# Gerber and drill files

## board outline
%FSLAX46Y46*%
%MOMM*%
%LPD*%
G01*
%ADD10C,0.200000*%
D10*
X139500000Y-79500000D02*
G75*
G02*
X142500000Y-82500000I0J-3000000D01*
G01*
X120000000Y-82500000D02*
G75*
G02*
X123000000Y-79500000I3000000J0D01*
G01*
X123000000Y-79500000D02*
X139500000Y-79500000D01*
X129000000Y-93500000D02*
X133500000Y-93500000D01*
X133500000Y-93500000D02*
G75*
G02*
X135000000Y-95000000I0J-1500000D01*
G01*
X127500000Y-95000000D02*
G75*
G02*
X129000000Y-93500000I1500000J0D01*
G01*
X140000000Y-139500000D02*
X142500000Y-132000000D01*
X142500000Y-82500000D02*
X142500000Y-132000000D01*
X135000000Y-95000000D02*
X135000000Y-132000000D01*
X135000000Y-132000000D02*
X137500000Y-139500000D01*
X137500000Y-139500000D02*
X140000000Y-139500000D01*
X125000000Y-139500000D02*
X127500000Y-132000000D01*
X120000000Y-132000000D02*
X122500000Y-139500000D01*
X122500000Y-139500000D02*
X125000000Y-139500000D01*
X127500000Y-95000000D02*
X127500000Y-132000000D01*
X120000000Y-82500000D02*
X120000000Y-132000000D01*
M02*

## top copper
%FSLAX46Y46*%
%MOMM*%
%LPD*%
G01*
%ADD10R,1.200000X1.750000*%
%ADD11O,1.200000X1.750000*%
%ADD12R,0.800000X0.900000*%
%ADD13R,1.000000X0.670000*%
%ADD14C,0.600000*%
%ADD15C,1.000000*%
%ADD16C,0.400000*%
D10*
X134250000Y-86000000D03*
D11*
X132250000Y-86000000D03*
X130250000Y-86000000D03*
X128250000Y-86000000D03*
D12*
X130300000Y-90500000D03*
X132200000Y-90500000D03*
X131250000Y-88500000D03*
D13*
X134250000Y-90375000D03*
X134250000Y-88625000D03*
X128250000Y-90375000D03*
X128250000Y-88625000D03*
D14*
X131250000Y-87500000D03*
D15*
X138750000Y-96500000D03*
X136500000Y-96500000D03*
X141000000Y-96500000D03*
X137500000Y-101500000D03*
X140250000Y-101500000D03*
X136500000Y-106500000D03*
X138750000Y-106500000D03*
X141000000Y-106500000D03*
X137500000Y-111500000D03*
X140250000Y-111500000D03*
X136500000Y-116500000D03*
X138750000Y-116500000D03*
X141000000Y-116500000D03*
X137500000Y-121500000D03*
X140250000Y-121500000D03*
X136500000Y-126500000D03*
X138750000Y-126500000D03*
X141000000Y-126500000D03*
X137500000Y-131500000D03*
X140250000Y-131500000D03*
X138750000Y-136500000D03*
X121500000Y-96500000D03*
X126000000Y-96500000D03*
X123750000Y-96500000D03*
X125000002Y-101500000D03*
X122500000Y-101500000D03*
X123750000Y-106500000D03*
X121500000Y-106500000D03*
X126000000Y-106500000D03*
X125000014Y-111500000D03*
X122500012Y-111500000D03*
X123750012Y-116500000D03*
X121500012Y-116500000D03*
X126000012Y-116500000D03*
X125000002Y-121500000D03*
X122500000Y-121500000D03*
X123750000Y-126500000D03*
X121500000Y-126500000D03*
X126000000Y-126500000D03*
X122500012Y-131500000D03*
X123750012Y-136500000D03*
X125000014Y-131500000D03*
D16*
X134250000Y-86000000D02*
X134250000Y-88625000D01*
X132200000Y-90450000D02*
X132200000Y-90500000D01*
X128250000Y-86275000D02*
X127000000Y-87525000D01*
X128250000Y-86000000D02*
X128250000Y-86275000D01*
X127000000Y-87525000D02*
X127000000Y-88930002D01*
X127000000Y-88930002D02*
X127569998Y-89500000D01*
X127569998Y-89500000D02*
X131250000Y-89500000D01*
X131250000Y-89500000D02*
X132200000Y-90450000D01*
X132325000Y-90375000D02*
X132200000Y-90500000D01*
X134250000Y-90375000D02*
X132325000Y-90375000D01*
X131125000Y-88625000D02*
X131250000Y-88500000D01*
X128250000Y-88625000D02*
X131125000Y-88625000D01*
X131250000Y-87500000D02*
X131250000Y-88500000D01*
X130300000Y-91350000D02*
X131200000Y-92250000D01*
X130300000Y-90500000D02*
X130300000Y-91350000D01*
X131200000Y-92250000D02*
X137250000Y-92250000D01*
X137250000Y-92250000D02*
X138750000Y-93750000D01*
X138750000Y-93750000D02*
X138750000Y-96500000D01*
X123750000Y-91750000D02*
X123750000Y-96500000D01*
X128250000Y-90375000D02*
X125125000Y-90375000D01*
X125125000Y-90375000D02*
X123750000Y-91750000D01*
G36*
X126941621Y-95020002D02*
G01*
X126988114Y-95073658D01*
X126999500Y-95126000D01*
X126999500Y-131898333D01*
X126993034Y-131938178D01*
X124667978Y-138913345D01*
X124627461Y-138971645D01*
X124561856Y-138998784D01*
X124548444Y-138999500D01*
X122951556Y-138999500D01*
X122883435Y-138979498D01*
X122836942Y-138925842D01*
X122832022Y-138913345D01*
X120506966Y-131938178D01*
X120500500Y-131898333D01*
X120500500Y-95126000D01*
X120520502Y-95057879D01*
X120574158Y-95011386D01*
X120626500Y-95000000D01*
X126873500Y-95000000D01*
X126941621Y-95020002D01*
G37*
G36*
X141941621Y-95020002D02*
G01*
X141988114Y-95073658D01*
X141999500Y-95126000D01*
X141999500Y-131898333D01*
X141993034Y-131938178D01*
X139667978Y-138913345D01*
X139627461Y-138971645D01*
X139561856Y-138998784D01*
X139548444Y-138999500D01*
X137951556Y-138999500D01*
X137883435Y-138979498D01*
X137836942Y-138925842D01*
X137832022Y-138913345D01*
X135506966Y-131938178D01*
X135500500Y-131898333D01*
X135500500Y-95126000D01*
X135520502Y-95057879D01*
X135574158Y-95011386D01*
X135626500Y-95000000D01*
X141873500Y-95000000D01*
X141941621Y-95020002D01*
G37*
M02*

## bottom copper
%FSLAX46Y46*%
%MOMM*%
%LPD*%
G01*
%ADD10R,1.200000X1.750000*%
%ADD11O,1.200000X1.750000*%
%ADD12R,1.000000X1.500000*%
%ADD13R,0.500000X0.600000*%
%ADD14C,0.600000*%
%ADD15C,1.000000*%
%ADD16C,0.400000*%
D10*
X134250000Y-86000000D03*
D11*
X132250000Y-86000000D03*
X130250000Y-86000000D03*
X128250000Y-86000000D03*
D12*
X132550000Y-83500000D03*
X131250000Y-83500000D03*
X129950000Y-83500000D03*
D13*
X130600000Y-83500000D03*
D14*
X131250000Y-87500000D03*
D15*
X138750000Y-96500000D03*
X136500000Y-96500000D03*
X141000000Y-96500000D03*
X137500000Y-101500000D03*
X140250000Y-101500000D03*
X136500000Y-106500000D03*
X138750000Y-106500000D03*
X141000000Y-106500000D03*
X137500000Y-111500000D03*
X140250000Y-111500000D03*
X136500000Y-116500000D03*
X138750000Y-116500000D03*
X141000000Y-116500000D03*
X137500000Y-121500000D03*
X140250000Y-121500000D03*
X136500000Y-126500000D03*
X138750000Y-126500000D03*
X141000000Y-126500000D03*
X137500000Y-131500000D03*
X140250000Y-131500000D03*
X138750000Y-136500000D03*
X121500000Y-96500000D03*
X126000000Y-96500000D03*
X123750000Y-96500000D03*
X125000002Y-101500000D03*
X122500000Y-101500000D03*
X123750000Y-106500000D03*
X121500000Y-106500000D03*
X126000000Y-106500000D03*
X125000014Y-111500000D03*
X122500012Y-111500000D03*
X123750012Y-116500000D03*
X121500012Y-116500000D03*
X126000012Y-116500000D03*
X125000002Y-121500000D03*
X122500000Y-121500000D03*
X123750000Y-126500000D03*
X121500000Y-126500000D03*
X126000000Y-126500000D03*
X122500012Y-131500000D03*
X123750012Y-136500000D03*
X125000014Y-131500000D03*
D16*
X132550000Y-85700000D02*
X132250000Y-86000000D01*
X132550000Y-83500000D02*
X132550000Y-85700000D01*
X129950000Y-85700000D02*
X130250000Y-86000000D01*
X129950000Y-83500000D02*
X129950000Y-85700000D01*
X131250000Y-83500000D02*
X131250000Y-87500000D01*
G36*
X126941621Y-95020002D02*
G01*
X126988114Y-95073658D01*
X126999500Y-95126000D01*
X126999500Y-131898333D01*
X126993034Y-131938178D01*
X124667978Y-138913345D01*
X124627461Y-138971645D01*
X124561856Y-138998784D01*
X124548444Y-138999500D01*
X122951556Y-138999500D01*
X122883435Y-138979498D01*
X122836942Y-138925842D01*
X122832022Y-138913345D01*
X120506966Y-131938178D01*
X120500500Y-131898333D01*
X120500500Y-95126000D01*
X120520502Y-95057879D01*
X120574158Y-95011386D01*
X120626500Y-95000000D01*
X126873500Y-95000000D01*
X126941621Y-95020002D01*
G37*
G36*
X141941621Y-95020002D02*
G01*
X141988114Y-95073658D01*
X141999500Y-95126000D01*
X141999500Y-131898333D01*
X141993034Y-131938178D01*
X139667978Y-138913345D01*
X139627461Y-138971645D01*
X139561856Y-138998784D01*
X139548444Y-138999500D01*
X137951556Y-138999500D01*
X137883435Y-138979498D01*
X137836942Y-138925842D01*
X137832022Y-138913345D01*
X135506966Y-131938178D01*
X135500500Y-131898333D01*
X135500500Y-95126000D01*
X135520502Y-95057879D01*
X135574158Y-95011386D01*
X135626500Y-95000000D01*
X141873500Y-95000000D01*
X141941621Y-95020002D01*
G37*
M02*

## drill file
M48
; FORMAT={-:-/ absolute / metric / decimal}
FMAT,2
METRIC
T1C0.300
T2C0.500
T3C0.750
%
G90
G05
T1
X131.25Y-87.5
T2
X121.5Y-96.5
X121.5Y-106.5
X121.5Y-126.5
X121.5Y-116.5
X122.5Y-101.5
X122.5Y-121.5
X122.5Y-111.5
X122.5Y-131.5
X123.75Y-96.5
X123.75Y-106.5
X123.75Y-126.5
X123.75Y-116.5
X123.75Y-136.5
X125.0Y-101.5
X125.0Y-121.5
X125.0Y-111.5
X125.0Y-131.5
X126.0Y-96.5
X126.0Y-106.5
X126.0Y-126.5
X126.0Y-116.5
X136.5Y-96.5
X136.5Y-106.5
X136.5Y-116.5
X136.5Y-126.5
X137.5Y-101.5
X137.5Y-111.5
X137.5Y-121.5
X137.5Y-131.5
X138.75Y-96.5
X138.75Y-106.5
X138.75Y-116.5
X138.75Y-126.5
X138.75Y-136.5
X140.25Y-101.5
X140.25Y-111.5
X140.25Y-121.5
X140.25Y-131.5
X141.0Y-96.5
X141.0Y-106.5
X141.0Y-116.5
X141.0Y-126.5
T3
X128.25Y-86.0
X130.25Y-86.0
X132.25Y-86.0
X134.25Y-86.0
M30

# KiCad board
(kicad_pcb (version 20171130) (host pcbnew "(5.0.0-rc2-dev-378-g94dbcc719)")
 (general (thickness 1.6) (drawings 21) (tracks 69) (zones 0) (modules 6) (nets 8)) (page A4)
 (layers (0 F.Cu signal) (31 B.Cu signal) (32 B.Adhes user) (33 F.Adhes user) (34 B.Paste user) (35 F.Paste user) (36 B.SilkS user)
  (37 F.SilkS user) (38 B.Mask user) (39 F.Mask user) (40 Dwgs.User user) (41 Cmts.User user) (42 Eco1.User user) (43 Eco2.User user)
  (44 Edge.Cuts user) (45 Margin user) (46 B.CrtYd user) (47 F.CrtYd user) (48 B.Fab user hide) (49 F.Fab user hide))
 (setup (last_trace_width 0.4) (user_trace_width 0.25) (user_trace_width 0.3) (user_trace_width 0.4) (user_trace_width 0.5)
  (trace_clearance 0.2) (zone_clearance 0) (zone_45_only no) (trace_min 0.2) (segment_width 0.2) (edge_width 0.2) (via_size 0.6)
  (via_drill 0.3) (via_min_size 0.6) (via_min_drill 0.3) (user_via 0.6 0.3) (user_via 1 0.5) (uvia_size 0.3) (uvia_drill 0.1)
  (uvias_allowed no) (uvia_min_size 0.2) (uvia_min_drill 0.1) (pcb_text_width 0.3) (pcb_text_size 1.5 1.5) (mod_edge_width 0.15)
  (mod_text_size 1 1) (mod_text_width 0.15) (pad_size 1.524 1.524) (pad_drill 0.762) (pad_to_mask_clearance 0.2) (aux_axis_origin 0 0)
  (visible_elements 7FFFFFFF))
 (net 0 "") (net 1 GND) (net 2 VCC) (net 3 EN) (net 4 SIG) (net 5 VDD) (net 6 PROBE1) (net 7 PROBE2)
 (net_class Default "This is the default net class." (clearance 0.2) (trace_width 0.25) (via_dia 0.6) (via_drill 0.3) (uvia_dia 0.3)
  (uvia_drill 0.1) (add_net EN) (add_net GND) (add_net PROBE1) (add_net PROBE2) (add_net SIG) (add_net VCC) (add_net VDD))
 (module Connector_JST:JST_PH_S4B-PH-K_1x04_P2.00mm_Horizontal (layer F.Cu) (at 134.25 86 180)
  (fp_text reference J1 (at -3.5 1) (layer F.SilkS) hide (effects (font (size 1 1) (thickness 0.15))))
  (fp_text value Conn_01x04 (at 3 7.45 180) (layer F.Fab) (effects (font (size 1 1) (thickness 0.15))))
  (pad 1 thru_hole rect (at 0 0 180) (size 1.2 1.75) (drill 0.75) (layers *.Cu *.Mask) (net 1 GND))
  (pad 2 thru_hole oval (at 2 0 180) (size 1.2 1.75) (drill 0.75) (layers *.Cu *.Mask) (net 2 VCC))
  (pad 3 thru_hole oval (at 4 0 180) (size 1.2 1.75) (drill 0.75) (layers *.Cu *.Mask) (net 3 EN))
  (pad 4 thru_hole oval (at 6 0 180) (size 1.2 1.75) (drill 0.75) (layers *.Cu *.Mask) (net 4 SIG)))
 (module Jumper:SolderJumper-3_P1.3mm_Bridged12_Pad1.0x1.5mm (layer B.Cu) (at 131.25 83.5)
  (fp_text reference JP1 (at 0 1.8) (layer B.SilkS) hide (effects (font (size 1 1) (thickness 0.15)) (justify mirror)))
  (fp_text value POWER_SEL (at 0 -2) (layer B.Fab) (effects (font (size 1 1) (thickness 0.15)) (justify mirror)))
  (pad 3 smd rect (at 1.3 0) (size 1 1.5) (layers B.Cu B.Mask) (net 2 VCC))
  (pad 2 smd rect (at 0 0) (size 1 1.5) (layers B.Cu B.Mask) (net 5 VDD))
  (pad 1 smd rect (at -1.3 0) (size 1 1.5) (layers B.Cu B.Mask) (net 3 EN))
  (pad 1 smd rect (at -0.65 0) (size 0.5 0.6) (layers B.Cu B.Mask) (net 3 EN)))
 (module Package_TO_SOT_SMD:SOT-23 (layer F.Cu) (at 131.25 89.5 90)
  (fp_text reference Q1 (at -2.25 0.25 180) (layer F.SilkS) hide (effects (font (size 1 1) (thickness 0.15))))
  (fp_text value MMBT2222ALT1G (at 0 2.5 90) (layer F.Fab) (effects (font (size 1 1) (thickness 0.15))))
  (pad 1 smd rect (at -1 -0.95 90) (size 0.9 0.8) (layers F.Cu F.Paste F.Mask) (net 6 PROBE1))
  (pad 2 smd rect (at -1 0.95 90) (size 0.9 0.8) (layers F.Cu F.Paste F.Mask) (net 4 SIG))
  (pad 3 smd rect (at 1 0 90) (size 0.9 0.8) (layers F.Cu F.Paste F.Mask) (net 5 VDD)))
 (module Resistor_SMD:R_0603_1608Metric (layer F.Cu) (at 134.25 89.5 90)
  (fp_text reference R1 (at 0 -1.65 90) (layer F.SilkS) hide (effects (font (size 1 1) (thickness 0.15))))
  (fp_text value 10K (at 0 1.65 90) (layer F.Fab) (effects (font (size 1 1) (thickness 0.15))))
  (pad 1 smd rect (at -0.875 0 90) (size 0.67 1) (layers F.Cu F.Paste F.Mask) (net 4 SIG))
  (pad 2 smd rect (at 0.875 0 90) (size 0.67 1) (layers F.Cu F.Paste F.Mask) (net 1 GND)))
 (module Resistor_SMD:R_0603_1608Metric (layer F.Cu) (at 128.25 89.5 270)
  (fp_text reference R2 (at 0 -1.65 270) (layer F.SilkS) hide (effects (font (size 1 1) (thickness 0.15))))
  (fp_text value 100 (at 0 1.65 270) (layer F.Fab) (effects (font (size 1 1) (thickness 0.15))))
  (pad 2 smd rect (at 0.875 0 270) (size 0.67 1) (layers F.Cu F.Paste F.Mask) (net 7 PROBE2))
  (pad 1 smd rect (at -0.875 0 270) (size 0.67 1) (layers F.Cu F.Paste F.Mask) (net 5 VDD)))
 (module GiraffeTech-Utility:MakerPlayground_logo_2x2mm (layer F.Cu) (at 139.5 84.5)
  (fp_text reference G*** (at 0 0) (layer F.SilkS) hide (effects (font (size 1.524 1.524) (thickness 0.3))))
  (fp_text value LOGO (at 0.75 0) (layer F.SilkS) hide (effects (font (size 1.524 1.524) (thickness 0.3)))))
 (gr_arc (start 139.5 82.5) (end 142.5 82.5) (angle -90) (layer Edge.Cuts) (width 0.2))
 (gr_arc (start 123 82.5) (end 123 79.5) (angle -90) (layer Edge.Cuts) (width 0.2))
 (gr_line (start 123 79.5) (end 139.5 79.5) (layer Edge.Cuts) (width 0.2))
 (gr_line (start 129 93.5) (end 133.5 93.5) (layer Edge.Cuts) (width 0.2))
 (gr_arc (start 133.5 95) (end 135 95) (angle -90) (layer Edge.Cuts) (width 0.2))
 (gr_arc (start 129 95) (end 129 93.5) (angle -90) (layer Edge.Cuts) (width 0.2))
 (gr_line (start 140 139.5) (end 142.5 132) (layer Edge.Cuts) (width 0.2))
 (gr_line (start 142.5 82.5) (end 142.5 132) (layer Edge.Cuts) (width 0.2))
 (gr_line (start 135 95) (end 135 132) (layer Edge.Cuts) (width 0.2))
 (gr_line (start 135 132) (end 137.5 139.5) (layer Edge.Cuts) (width 0.2))
 (gr_line (start 137.5 139.5) (end 140 139.5) (layer Edge.Cuts) (width 0.2))
 (gr_line (start 125 139.5) (end 127.5 132) (layer Edge.Cuts) (width 0.2))
 (gr_line (start 120 132) (end 122.5 139.5) (layer Edge.Cuts) (width 0.2))
 (gr_line (start 122.5 139.5) (end 125 139.5) (layer Edge.Cuts) (width 0.2))
 (gr_line (start 127.5 95) (end 127.5 132) (layer Edge.Cuts) (width 0.2))
 (gr_line (start 120 82.5) (end 120 132) (layer Edge.Cuts) (width 0.2))
 (segment (start 134.25 86) (end 134.25 88.625) (width 0.4) (layer F.Cu) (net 1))
 (segment (start 132.55 85.7) (end 132.25 86) (width 0.4) (layer B.Cu) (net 2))
 (segment (start 132.55 83.5) (end 132.55 85.7) (width 0.4) (layer B.Cu) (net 2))
 (segment (start 129.95 85.7) (end 130.25 86) (width 0.4) (layer B.Cu) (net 3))
 (segment (start 129.95 83.5) (end 129.95 85.7) (width 0.4) (layer B.Cu) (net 3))
 (segment (start 132.2 90.45) (end 132.2 90.5) (width 0.4) (layer F.Cu) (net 4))
 (segment (start 128.25 86.275) (end 127 87.525) (width 0.4) (layer F.Cu) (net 4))
 (segment (start 128.25 86) (end 128.25 86.275) (width 0.4) (layer F.Cu) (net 4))
 (segment (start 127 87.525) (end 127 88.930002) (width 0.4) (layer F.Cu) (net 4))
 (segment (start 127 88.930002) (end 127.569998 89.5) (width 0.4) (layer F.Cu) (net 4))
 (segment (start 127.569998 89.5) (end 131.25 89.5) (width 0.4) (layer F.Cu) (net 4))
 (segment (start 131.25 89.5) (end 132.2 90.45) (width 0.4) (layer F.Cu) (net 4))
 (segment (start 132.325 90.375) (end 132.2 90.5) (width 0.4) (layer F.Cu) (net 4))
 (segment (start 134.25 90.375) (end 132.325 90.375) (width 0.4) (layer F.Cu) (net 4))
 (segment (start 131.125 88.625) (end 131.25 88.5) (width 0.4) (layer F.Cu) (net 5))
 (segment (start 128.25 88.625) (end 131.125 88.625) (width 0.4) (layer F.Cu) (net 5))
 (via (at 131.25 87.5) (size 0.6) (drill 0.3) (layers F.Cu B.Cu) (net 5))
 (segment (start 131.25 83.5) (end 131.25 87.5) (width 0.4) (layer B.Cu) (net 5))
 (segment (start 131.25 87.5) (end 131.25 88.5) (width 0.4) (layer F.Cu) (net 5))
 (segment (start 130.3 91.35) (end 131.2 92.25) (width 0.4) (layer F.Cu) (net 6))
 (segment (start 130.3 90.5) (end 130.3 91.35) (width 0.4) (layer F.Cu) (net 6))
 (segment (start 131.2 92.25) (end 137.25 92.25) (width 0.4) (layer F.Cu) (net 6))
 (via (at 138.75 96.5) (size 1) (drill 0.5) (layers F.Cu B.Cu) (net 6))
 (segment (start 137.25 92.25) (end 138.75 93.75) (width 0.4) (layer F.Cu) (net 6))
 (segment (start 138.75 93.75) (end 138.75 96.5) (width 0.4) (layer F.Cu) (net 6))
 (via (at 136.5 96.5) (size 1) (drill 0.5) (layers F.Cu B.Cu) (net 6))
 (via (at 141 96.5) (size 1) (drill 0.5) (layers F.Cu B.Cu) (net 6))
 (via (at 137.5 101.5) (size 1) (drill 0.5) (layers F.Cu B.Cu) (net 6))
 (via (at 140.25 101.5) (size 1) (drill 0.5) (layers F.Cu B.Cu) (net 6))
 (via (at 136.5 106.5) (size 1) (drill 0.5) (layers F.Cu B.Cu) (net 6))
 (via (at 138.75 106.5) (size 1) (drill 0.5) (layers F.Cu B.Cu) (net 6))
 (via (at 141 106.5) (size 1) (drill 0.5) (layers F.Cu B.Cu) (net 6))
 (via (at 137.5 111.5) (size 1) (drill 0.5) (layers F.Cu B.Cu) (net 6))
 (via (at 140.25 111.5) (size 1) (drill 0.5) (layers F.Cu B.Cu) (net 6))
 (via (at 136.5 116.5) (size 1) (drill 0.5) (layers F.Cu B.Cu) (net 6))
 (via (at 138.75 116.5) (size 1) (drill 0.5) (layers F.Cu B.Cu) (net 6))
 (via (at 141 116.5) (size 1) (drill 0.5) (layers F.Cu B.Cu) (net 6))
 (via (at 137.5 121.5) (size 1) (drill 0.5) (layers F.Cu B.Cu) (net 6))
 (via (at 140.25 121.5) (size 1) (drill 0.5) (layers F.Cu B.Cu) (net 6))
 (via (at 136.5 126.5) (size 1) (drill 0.5) (layers F.Cu B.Cu) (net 6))
 (via (at 138.75 126.5) (size 1) (drill 0.5) (layers F.Cu B.Cu) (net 6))
 (via (at 141 126.5) (size 1) (drill 0.5) (layers F.Cu B.Cu) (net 6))
 (via (at 137.5 131.5) (size 1) (drill 0.5) (layers F.Cu B.Cu) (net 6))
 (via (at 140.25 131.5) (size 1) (drill 0.5) (layers F.Cu B.Cu) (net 6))
 (via (at 138.75 136.5) (size 1) (drill 0.5) (layers F.Cu B.Cu) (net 6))
 (via (at 121.5 96.5) (size 1) (drill 0.5) (layers F.Cu B.Cu) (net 7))
 (via (at 126 96.5) (size 1) (drill 0.5) (layers F.Cu B.Cu) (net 7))
 (via (at 123.75 96.5) (size 1) (drill 0.5) (layers F.Cu B.Cu) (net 7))
 (segment (start 123.75 91.75) (end 123.75 96.5) (width 0.4) (layer F.Cu) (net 7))
 (segment (start 128.25 90.375) (end 125.125 90.375) (width 0.4) (layer F.Cu) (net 7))
 (segment (start 125.125 90.375) (end 123.75 91.75) (width 0.4) (layer F.Cu) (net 7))
 (via (at 125.000002 101.5) (size 1) (drill 0.5) (layers F.Cu B.Cu) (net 7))
 (via (at 122.5 101.5) (size 1) (drill 0.5) (layers F.Cu B.Cu) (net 7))
 (via (at 123.75 106.5) (size 1) (drill 0.5) (layers F.Cu B.Cu) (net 7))
 (via (at 121.5 106.5) (size 1) (drill 0.5) (layers F.Cu B.Cu) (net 7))
 (via (at 126 106.5) (size 1) (drill 0.5) (layers F.Cu B.Cu) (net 7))
 (via (at 125.000014 111.5) (size 1) (drill 0.5) (layers F.Cu B.Cu) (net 7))
 (via (at 122.500012 111.5) (size 1) (drill 0.5) (layers F.Cu B.Cu) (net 7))
 (via (at 123.750012 116.5) (size 1) (drill 0.5) (layers F.Cu B.Cu) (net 7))
 (via (at 121.500012 116.5) (size 1) (drill 0.5) (layers F.Cu B.Cu) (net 7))
 (via (at 126.000012 116.5) (size 1) (drill 0.5) (layers F.Cu B.Cu) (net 7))
 (via (at 125.000002 121.5) (size 1) (drill 0.5) (layers F.Cu B.Cu) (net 7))
 (via (at 122.5 121.5) (size 1) (drill 0.5) (layers F.Cu B.Cu) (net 7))
 (via (at 123.75 126.5) (size 1) (drill 0.5) (layers F.Cu B.Cu) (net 7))
 (via (at 121.5 126.5) (size 1) (drill 0.5) (layers F.Cu B.Cu) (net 7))
 (via (at 126 126.5) (size 1) (drill 0.5) (layers F.Cu B.Cu) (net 7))
 (via (at 122.500012 131.5) (size 1) (drill 0.5) (layers F.Cu B.Cu) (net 7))
 (via (at 123.750012 136.5) (size 1) (drill 0.5) (layers F.Cu B.Cu) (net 7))
 (via (at 125.000014 131.5) (size 1) (drill 0.5) (layers F.Cu B.Cu) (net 7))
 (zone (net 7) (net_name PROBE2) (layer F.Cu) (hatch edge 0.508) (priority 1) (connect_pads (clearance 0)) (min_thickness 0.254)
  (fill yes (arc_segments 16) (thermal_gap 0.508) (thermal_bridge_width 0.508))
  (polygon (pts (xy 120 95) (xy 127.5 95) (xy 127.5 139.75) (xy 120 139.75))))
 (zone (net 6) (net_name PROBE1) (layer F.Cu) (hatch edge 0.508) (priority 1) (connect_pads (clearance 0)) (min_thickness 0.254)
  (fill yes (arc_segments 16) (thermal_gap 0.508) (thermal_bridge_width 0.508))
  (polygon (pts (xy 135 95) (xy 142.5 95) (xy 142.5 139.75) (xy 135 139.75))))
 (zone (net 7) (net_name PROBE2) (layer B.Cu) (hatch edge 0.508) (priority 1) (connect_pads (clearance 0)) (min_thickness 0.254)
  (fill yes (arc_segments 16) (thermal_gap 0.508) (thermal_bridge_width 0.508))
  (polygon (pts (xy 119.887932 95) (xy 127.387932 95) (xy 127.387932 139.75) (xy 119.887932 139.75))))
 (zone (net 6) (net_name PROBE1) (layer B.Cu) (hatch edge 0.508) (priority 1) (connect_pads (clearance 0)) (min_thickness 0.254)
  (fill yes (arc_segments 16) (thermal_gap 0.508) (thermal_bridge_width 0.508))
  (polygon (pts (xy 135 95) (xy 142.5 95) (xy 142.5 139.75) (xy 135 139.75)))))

